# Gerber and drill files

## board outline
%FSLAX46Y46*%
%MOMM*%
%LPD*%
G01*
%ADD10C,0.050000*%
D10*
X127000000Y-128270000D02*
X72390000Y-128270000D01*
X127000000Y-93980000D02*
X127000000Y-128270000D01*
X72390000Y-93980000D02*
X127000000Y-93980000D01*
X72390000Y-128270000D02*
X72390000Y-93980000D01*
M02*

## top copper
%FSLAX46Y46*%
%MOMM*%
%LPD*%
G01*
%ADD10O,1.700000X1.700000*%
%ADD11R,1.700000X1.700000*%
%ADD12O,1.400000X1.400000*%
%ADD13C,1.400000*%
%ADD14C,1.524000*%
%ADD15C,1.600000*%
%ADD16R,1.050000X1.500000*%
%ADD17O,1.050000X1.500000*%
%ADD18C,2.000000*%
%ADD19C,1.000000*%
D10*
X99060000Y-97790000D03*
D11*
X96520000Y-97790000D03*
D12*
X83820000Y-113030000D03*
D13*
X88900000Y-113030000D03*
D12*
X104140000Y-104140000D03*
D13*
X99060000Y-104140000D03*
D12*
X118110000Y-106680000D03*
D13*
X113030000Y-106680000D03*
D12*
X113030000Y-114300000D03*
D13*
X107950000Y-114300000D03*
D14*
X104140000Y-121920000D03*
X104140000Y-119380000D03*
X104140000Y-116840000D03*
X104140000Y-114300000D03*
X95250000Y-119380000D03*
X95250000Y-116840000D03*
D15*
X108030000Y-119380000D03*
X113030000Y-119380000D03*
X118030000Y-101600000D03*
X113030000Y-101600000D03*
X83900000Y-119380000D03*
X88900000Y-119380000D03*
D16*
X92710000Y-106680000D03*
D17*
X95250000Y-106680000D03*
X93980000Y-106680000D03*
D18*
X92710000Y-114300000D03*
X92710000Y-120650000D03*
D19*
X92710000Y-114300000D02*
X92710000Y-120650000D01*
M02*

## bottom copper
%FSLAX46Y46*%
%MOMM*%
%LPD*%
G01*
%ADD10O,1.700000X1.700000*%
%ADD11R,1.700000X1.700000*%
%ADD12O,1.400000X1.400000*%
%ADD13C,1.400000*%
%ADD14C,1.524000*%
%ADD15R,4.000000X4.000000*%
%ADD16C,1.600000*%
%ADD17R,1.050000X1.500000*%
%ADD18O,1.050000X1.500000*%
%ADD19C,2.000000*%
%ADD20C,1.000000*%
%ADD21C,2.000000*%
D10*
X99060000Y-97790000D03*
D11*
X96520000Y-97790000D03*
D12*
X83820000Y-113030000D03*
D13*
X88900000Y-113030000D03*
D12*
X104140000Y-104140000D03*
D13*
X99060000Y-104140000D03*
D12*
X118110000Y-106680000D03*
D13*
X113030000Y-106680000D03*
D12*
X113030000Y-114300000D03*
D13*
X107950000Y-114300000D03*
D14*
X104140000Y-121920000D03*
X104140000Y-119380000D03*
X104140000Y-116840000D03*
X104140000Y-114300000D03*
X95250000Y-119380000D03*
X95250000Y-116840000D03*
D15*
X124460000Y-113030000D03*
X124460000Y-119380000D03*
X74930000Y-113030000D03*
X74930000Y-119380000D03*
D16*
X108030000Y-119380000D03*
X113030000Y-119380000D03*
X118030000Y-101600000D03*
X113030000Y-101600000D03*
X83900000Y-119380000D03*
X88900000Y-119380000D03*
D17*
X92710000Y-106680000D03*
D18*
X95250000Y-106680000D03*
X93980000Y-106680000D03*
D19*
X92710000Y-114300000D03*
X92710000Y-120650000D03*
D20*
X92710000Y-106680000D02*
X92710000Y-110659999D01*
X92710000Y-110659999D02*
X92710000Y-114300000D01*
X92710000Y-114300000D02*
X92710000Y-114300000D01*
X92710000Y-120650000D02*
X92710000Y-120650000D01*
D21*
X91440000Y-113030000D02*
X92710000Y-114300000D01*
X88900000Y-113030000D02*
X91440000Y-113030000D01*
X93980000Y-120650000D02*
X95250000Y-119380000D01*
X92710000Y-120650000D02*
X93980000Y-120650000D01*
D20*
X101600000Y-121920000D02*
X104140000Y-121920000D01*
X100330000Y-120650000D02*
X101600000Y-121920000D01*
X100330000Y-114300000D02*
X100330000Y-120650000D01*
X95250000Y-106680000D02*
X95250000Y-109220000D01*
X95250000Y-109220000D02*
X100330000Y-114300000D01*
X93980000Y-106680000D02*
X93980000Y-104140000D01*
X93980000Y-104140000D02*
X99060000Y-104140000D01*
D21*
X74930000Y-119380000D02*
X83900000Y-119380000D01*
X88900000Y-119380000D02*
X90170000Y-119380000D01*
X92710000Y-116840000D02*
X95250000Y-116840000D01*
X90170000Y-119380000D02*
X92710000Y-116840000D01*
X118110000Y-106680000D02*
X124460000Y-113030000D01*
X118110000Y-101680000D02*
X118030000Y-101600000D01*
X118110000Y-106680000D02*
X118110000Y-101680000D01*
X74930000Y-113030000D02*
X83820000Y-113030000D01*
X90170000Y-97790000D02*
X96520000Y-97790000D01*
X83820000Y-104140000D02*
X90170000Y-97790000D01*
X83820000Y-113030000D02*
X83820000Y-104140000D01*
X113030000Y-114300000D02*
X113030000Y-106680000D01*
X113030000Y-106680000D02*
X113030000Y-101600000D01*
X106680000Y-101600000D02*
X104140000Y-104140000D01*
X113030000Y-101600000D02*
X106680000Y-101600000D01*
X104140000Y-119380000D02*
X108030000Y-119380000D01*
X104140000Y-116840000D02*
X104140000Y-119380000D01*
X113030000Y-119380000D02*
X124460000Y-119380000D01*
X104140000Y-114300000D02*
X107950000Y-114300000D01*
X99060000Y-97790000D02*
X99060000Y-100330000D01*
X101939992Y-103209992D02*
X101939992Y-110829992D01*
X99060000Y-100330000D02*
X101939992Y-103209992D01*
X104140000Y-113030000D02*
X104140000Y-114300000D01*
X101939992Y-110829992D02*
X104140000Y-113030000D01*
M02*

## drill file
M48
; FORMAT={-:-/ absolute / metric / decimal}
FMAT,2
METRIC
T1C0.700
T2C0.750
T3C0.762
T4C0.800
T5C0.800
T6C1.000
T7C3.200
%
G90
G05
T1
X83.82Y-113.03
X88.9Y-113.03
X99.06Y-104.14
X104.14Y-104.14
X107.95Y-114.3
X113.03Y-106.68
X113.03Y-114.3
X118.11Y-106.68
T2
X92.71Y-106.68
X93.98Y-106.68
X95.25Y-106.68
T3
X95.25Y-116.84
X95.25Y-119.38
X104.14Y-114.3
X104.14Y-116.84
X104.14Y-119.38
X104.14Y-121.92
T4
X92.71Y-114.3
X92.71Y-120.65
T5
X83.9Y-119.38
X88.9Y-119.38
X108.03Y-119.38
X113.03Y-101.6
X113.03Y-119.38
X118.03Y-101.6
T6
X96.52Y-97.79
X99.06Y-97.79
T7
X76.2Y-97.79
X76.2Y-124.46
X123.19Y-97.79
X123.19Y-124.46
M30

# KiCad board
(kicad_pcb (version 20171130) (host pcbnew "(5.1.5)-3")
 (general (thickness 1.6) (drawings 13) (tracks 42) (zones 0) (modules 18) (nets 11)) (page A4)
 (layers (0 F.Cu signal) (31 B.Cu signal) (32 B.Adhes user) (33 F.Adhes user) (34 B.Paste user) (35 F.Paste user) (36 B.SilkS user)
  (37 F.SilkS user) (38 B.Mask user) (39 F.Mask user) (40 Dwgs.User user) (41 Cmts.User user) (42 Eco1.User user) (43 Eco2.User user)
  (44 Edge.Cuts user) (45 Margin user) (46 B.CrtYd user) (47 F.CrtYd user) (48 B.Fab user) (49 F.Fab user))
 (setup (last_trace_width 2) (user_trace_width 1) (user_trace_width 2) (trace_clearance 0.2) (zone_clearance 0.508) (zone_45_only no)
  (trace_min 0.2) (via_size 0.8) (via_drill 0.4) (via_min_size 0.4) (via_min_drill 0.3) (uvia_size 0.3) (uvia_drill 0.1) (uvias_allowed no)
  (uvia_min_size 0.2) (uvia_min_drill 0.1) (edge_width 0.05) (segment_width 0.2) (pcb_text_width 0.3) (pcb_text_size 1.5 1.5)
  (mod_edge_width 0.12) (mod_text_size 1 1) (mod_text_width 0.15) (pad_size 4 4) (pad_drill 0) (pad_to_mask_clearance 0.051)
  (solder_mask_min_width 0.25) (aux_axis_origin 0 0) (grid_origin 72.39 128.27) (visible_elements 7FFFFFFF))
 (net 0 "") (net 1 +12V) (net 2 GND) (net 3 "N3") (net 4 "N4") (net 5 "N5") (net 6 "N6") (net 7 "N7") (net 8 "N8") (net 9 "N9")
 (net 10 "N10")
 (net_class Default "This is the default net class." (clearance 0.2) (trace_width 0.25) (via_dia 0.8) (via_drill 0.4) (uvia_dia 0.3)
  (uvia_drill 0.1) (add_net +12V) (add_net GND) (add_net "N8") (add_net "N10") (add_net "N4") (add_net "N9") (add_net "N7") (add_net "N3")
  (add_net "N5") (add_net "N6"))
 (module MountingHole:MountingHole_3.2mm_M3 (layer F.Cu) (at 123.19 124.46)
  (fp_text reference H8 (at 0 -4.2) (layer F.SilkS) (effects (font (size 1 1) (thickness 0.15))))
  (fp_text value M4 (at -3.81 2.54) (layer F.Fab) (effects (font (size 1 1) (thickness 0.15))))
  (pad 1 np_thru_hole circle (at 0 0) (size 3.2 3.2) (drill 3.2) (layers *.Cu *.Mask)))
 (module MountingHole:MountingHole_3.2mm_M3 (layer F.Cu) (at 123.19 97.79)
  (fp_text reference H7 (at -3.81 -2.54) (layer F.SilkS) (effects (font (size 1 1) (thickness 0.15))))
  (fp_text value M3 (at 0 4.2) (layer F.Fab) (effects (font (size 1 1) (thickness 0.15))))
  (pad 1 np_thru_hole circle (at 0 0) (size 3.2 3.2) (drill 3.2) (layers *.Cu *.Mask)))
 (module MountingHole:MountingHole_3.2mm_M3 (layer F.Cu) (at 76.2 124.46)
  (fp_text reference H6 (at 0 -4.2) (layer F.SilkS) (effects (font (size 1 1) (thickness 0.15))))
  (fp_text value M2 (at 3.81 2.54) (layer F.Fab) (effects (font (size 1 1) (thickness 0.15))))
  (pad 1 np_thru_hole circle (at 0 0) (size 3.2 3.2) (drill 3.2) (layers *.Cu *.Mask)))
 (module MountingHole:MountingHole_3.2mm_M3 (layer F.Cu) (at 76.2 97.79)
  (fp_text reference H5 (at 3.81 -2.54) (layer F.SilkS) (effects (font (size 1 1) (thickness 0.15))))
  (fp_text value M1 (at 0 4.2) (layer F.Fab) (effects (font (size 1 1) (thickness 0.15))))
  (pad 1 np_thru_hole circle (at 0 0) (size 3.2 3.2) (drill 3.2) (layers *.Cu *.Mask)))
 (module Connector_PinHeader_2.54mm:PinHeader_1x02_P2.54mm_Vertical (layer F.Cu) (at 96.52 97.79 90)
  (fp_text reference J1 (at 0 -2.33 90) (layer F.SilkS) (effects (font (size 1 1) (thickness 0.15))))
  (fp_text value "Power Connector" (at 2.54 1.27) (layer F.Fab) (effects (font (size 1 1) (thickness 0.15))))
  (pad 2 thru_hole oval (at 0 2.54 90) (size 1.7 1.7) (drill 1) (layers *.Cu *.Mask) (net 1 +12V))
  (pad 1 thru_hole rect (at 0 0 90) (size 1.7 1.7) (drill 1) (layers *.Cu *.Mask) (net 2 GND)))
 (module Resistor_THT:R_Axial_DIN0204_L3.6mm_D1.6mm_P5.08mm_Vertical (layer F.Cu) (at 88.9 113.03 180)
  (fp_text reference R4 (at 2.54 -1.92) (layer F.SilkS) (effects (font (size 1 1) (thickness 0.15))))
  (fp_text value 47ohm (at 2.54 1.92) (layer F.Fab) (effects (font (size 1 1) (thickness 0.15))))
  (pad 2 thru_hole oval (at 5.08 0 180) (size 1.4 1.4) (drill 0.7) (layers *.Cu *.Mask) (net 2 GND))
  (pad 1 thru_hole circle (at 0 0 180) (size 1.4 1.4) (drill 0.7) (layers *.Cu *.Mask) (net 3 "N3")))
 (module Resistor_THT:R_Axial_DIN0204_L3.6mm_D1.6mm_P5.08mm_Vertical (layer F.Cu) (at 99.06 104.14)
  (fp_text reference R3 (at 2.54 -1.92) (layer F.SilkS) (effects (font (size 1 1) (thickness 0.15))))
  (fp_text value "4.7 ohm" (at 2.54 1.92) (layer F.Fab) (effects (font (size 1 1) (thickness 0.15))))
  (pad 2 thru_hole oval (at 5.08 0) (size 1.4 1.4) (drill 0.7) (layers *.Cu *.Mask) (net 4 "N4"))
  (pad 1 thru_hole circle (at 0 0) (size 1.4 1.4) (drill 0.7) (layers *.Cu *.Mask) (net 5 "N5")))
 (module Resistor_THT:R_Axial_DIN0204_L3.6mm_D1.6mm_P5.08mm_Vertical (layer F.Cu) (at 113.03 106.68)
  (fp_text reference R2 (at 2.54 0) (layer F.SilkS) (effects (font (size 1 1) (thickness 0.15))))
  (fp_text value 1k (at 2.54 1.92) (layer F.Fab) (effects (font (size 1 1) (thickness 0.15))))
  (pad 2 thru_hole oval (at 5.08 0) (size 1.4 1.4) (drill 0.7) (layers *.Cu *.Mask) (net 2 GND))
  (pad 1 thru_hole circle (at 0 0) (size 1.4 1.4) (drill 0.7) (layers *.Cu *.Mask) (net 4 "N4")))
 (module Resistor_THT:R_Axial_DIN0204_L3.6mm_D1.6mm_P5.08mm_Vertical (layer F.Cu) (at 107.95 114.3)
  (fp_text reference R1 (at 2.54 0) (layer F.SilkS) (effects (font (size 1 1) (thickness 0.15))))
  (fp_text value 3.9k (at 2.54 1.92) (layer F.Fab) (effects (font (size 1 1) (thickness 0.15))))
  (pad 2 thru_hole oval (at 5.08 0) (size 1.4 1.4) (drill 0.7) (layers *.Cu *.Mask) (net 4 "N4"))
  (pad 1 thru_hole circle (at 0 0) (size 1.4 1.4) (drill 0.7) (layers *.Cu *.Mask) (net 1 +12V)))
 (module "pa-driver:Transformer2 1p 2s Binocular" (layer F.Cu) (at 100.33 118.11)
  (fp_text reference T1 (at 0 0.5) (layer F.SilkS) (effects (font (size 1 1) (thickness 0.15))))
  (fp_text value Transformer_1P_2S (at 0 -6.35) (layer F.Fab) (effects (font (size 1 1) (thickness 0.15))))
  (pad 6 thru_hole circle (at 3.81 3.81) (size 1.524 1.524) (drill 0.762) (layers *.Cu *.Mask) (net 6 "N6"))
  (pad 5 thru_hole circle (at 3.81 1.27) (size 1.524 1.524) (drill 0.762) (layers *.Cu *.Mask) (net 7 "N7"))
  (pad 4 thru_hole circle (at 3.81 -1.27) (size 1.524 1.524) (drill 0.762) (layers *.Cu *.Mask) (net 7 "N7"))
  (pad 3 thru_hole circle (at 3.81 -3.81) (size 1.524 1.524) (drill 0.762) (layers *.Cu *.Mask) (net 1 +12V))
  (pad 2 thru_hole circle (at -5.08 1.27) (size 1.524 1.524) (drill 0.762) (layers *.Cu *.Mask) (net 3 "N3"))
  (pad 1 thru_hole circle (at -5.08 -1.27) (size 1.524 1.524) (drill 0.762) (layers *.Cu *.Mask) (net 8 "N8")))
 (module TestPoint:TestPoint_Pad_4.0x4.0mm (layer F.Cu) (at 124.46 113.03)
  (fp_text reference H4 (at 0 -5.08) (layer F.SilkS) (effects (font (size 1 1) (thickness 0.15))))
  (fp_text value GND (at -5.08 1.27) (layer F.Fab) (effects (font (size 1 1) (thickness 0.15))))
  (pad 1 smd rect (at 0 0) (size 4 4) (layers B.Cu B.Mask) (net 2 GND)))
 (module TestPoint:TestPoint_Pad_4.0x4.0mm (layer F.Cu) (at 124.46 119.38)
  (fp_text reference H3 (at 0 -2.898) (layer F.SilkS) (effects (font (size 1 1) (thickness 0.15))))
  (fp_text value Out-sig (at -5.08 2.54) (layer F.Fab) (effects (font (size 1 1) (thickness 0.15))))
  (pad 1 smd rect (at 0 0) (size 4 4) (layers B.Cu B.Mask) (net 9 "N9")))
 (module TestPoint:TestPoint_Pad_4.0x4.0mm (layer F.Cu) (at 74.93 113.03)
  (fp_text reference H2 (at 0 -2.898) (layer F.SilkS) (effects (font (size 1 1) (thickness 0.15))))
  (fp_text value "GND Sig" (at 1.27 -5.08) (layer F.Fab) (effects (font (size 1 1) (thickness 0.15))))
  (pad 1 smd rect (at 0 0) (size 4 4) (layers B.Cu B.Mask) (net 2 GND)))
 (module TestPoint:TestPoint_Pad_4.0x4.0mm (layer F.Cu) (at 74.93 119.38)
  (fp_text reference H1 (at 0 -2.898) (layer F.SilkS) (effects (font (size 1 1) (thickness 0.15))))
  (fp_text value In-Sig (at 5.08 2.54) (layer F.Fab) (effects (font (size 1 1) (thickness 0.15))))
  (pad 1 smd rect (at 0 0) (size 4 4) (layers B.Cu B.Mask) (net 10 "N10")))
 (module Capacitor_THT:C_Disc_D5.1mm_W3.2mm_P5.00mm (layer F.Cu) (at 113.03 119.38 180)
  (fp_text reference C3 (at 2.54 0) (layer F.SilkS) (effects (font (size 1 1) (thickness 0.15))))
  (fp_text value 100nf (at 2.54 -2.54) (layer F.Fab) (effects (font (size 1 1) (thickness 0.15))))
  (pad 2 thru_hole circle (at 5 0 180) (size 1.6 1.6) (drill 0.8) (layers *.Cu *.Mask) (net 7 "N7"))
  (pad 1 thru_hole circle (at 0 0 180) (size 1.6 1.6) (drill 0.8) (layers *.Cu *.Mask) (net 9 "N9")))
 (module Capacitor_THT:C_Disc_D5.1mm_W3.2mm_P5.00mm (layer F.Cu) (at 113.03 101.6)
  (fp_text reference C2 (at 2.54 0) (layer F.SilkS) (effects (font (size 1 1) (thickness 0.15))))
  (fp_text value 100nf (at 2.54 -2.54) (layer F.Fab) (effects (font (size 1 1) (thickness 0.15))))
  (pad 2 thru_hole circle (at 5 0) (size 1.6 1.6) (drill 0.8) (layers *.Cu *.Mask) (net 2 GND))
  (pad 1 thru_hole circle (at 0 0) (size 1.6 1.6) (drill 0.8) (layers *.Cu *.Mask) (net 4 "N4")))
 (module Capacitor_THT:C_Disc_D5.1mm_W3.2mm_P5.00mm (layer F.Cu) (at 88.9 119.38 180)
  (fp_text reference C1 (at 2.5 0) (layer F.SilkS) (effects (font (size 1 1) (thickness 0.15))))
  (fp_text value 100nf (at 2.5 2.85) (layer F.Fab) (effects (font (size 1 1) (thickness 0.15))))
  (pad 2 thru_hole circle (at 5 0 180) (size 1.6 1.6) (drill 0.8) (layers *.Cu *.Mask) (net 10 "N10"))
  (pad 1 thru_hole circle (at 0 0 180) (size 1.6 1.6) (drill 0.8) (layers *.Cu *.Mask) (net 8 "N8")))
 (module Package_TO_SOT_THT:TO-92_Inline (layer F.Cu) (at 92.71 106.68)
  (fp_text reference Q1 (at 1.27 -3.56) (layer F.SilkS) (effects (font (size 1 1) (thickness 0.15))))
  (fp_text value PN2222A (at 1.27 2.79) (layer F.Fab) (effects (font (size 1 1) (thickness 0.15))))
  (pad 1 thru_hole rect (at 0 0) (size 1.05 1.5) (drill 0.75) (layers *.Cu *.Mask) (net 3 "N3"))
  (pad 3 thru_hole oval (at 2.54 0) (size 1.05 1.5) (drill 0.75) (layers *.Cu *.Mask) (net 6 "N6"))
  (pad 2 thru_hole oval (at 1.27 0) (size 1.05 1.5) (drill 0.75) (layers *.Cu *.Mask) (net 5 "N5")))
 (gr_line (start 127 128.27) (end 72.39 128.27) (layer Edge.Cuts) (width 0.05))
 (gr_line (start 127 93.98) (end 127 128.27) (layer Edge.Cuts) (width 0.05))
 (gr_line (start 72.39 93.98) (end 127 93.98) (layer Edge.Cuts) (width 0.05))
 (gr_line (start 72.39 128.27) (end 72.39 93.98) (layer Edge.Cuts) (width 0.05))
 (segment (start 92.71 106.68) (end 92.71 110.659999) (width 1) (layer B.Cu) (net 3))
 (segment (start 92.71 110.659999) (end 92.71 114.3) (width 1) (layer B.Cu) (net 3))
 (segment (start 92.71 114.3) (end 92.71 114.3) (width 1) (layer B.Cu) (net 3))
 (via (at 92.71 114.3) (size 2) (drill 0.8) (layers F.Cu B.Cu) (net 3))
 (segment (start 92.71 120.65) (end 92.71 120.65) (width 1) (layer B.Cu) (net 3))
 (via (at 92.71 120.65) (size 2) (drill 0.8) (layers F.Cu B.Cu) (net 3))
 (segment (start 92.71 114.3) (end 92.71 120.65) (width 1) (layer F.Cu) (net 3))
 (segment (start 91.44 113.03) (end 92.71 114.3) (width 2) (layer B.Cu) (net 3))
 (segment (start 88.9 113.03) (end 91.44 113.03) (width 2) (layer B.Cu) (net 3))
 (segment (start 93.98 120.65) (end 95.25 119.38) (width 2) (layer B.Cu) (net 3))
 (segment (start 92.71 120.65) (end 93.98 120.65) (width 2) (layer B.Cu) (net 3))
 (segment (start 101.6 121.92) (end 104.14 121.92) (width 1) (layer B.Cu) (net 6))
 (segment (start 100.33 120.65) (end 101.6 121.92) (width 1) (layer B.Cu) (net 6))
 (segment (start 100.33 114.3) (end 100.33 120.65) (width 1) (layer B.Cu) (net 6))
 (segment (start 95.25 106.68) (end 95.25 109.22) (width 1) (layer B.Cu) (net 6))
 (segment (start 95.25 109.22) (end 100.33 114.3) (width 1) (layer B.Cu) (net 6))
 (segment (start 93.98 106.68) (end 93.98 104.14) (width 1) (layer B.Cu) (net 5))
 (segment (start 93.98 104.14) (end 99.06 104.14) (width 1) (layer B.Cu) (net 5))
 (segment (start 74.93 119.38) (end 83.9 119.38) (width 2) (layer B.Cu) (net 10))
 (segment (start 88.9 119.38) (end 90.17 119.38) (width 2) (layer B.Cu) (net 8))
 (segment (start 92.71 116.84) (end 95.25 116.84) (width 2) (layer B.Cu) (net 8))
 (segment (start 90.17 119.38) (end 92.71 116.84) (width 2) (layer B.Cu) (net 8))
 (segment (start 118.11 106.68) (end 124.46 113.03) (width 2) (layer B.Cu) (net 2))
 (segment (start 118.11 101.68) (end 118.03 101.6) (width 2) (layer B.Cu) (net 2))
 (segment (start 118.11 106.68) (end 118.11 101.68) (width 2) (layer B.Cu) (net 2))
 (segment (start 74.93 113.03) (end 83.82 113.03) (width 2) (layer B.Cu) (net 2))
 (segment (start 90.17 97.79) (end 96.52 97.79) (width 2) (layer B.Cu) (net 2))
 (segment (start 83.82 104.14) (end 90.17 97.79) (width 2) (layer B.Cu) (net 2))
 (segment (start 83.82 113.03) (end 83.82 104.14) (width 2) (layer B.Cu) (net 2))
 (segment (start 113.03 114.3) (end 113.03 106.68) (width 2) (layer B.Cu) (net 4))
 (segment (start 113.03 106.68) (end 113.03 101.6) (width 2) (layer B.Cu) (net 4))
 (segment (start 106.68 101.6) (end 104.14 104.14) (width 2) (layer B.Cu) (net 4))
 (segment (start 113.03 101.6) (end 106.68 101.6) (width 2) (layer B.Cu) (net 4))
 (segment (start 104.14 119.38) (end 108.03 119.38) (width 2) (layer B.Cu) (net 7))
 (segment (start 104.14 116.84) (end 104.14 119.38) (width 2) (layer B.Cu) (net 7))
 (segment (start 113.03 119.38) (end 124.46 119.38) (width 2) (layer B.Cu) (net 9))
 (segment (start 104.14 114.3) (end 107.95 114.3) (width 2) (layer B.Cu) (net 1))
 (segment (start 99.06 97.79) (end 99.06 100.33) (width 2) (layer B.Cu) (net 1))
 (segment (start 101.939992 103.209992) (end 101.939992 110.829992) (width 2) (layer B.Cu) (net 1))
 (segment (start 99.06 100.33) (end 101.939992 103.209992) (width 2) (layer B.Cu) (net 1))
 (segment (start 104.14 113.03) (end 104.14 114.3) (width 2) (layer B.Cu) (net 1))
 (segment (start 101.939992 110.829992) (end 104.14 113.03) (width 2) (layer B.Cu) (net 1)))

